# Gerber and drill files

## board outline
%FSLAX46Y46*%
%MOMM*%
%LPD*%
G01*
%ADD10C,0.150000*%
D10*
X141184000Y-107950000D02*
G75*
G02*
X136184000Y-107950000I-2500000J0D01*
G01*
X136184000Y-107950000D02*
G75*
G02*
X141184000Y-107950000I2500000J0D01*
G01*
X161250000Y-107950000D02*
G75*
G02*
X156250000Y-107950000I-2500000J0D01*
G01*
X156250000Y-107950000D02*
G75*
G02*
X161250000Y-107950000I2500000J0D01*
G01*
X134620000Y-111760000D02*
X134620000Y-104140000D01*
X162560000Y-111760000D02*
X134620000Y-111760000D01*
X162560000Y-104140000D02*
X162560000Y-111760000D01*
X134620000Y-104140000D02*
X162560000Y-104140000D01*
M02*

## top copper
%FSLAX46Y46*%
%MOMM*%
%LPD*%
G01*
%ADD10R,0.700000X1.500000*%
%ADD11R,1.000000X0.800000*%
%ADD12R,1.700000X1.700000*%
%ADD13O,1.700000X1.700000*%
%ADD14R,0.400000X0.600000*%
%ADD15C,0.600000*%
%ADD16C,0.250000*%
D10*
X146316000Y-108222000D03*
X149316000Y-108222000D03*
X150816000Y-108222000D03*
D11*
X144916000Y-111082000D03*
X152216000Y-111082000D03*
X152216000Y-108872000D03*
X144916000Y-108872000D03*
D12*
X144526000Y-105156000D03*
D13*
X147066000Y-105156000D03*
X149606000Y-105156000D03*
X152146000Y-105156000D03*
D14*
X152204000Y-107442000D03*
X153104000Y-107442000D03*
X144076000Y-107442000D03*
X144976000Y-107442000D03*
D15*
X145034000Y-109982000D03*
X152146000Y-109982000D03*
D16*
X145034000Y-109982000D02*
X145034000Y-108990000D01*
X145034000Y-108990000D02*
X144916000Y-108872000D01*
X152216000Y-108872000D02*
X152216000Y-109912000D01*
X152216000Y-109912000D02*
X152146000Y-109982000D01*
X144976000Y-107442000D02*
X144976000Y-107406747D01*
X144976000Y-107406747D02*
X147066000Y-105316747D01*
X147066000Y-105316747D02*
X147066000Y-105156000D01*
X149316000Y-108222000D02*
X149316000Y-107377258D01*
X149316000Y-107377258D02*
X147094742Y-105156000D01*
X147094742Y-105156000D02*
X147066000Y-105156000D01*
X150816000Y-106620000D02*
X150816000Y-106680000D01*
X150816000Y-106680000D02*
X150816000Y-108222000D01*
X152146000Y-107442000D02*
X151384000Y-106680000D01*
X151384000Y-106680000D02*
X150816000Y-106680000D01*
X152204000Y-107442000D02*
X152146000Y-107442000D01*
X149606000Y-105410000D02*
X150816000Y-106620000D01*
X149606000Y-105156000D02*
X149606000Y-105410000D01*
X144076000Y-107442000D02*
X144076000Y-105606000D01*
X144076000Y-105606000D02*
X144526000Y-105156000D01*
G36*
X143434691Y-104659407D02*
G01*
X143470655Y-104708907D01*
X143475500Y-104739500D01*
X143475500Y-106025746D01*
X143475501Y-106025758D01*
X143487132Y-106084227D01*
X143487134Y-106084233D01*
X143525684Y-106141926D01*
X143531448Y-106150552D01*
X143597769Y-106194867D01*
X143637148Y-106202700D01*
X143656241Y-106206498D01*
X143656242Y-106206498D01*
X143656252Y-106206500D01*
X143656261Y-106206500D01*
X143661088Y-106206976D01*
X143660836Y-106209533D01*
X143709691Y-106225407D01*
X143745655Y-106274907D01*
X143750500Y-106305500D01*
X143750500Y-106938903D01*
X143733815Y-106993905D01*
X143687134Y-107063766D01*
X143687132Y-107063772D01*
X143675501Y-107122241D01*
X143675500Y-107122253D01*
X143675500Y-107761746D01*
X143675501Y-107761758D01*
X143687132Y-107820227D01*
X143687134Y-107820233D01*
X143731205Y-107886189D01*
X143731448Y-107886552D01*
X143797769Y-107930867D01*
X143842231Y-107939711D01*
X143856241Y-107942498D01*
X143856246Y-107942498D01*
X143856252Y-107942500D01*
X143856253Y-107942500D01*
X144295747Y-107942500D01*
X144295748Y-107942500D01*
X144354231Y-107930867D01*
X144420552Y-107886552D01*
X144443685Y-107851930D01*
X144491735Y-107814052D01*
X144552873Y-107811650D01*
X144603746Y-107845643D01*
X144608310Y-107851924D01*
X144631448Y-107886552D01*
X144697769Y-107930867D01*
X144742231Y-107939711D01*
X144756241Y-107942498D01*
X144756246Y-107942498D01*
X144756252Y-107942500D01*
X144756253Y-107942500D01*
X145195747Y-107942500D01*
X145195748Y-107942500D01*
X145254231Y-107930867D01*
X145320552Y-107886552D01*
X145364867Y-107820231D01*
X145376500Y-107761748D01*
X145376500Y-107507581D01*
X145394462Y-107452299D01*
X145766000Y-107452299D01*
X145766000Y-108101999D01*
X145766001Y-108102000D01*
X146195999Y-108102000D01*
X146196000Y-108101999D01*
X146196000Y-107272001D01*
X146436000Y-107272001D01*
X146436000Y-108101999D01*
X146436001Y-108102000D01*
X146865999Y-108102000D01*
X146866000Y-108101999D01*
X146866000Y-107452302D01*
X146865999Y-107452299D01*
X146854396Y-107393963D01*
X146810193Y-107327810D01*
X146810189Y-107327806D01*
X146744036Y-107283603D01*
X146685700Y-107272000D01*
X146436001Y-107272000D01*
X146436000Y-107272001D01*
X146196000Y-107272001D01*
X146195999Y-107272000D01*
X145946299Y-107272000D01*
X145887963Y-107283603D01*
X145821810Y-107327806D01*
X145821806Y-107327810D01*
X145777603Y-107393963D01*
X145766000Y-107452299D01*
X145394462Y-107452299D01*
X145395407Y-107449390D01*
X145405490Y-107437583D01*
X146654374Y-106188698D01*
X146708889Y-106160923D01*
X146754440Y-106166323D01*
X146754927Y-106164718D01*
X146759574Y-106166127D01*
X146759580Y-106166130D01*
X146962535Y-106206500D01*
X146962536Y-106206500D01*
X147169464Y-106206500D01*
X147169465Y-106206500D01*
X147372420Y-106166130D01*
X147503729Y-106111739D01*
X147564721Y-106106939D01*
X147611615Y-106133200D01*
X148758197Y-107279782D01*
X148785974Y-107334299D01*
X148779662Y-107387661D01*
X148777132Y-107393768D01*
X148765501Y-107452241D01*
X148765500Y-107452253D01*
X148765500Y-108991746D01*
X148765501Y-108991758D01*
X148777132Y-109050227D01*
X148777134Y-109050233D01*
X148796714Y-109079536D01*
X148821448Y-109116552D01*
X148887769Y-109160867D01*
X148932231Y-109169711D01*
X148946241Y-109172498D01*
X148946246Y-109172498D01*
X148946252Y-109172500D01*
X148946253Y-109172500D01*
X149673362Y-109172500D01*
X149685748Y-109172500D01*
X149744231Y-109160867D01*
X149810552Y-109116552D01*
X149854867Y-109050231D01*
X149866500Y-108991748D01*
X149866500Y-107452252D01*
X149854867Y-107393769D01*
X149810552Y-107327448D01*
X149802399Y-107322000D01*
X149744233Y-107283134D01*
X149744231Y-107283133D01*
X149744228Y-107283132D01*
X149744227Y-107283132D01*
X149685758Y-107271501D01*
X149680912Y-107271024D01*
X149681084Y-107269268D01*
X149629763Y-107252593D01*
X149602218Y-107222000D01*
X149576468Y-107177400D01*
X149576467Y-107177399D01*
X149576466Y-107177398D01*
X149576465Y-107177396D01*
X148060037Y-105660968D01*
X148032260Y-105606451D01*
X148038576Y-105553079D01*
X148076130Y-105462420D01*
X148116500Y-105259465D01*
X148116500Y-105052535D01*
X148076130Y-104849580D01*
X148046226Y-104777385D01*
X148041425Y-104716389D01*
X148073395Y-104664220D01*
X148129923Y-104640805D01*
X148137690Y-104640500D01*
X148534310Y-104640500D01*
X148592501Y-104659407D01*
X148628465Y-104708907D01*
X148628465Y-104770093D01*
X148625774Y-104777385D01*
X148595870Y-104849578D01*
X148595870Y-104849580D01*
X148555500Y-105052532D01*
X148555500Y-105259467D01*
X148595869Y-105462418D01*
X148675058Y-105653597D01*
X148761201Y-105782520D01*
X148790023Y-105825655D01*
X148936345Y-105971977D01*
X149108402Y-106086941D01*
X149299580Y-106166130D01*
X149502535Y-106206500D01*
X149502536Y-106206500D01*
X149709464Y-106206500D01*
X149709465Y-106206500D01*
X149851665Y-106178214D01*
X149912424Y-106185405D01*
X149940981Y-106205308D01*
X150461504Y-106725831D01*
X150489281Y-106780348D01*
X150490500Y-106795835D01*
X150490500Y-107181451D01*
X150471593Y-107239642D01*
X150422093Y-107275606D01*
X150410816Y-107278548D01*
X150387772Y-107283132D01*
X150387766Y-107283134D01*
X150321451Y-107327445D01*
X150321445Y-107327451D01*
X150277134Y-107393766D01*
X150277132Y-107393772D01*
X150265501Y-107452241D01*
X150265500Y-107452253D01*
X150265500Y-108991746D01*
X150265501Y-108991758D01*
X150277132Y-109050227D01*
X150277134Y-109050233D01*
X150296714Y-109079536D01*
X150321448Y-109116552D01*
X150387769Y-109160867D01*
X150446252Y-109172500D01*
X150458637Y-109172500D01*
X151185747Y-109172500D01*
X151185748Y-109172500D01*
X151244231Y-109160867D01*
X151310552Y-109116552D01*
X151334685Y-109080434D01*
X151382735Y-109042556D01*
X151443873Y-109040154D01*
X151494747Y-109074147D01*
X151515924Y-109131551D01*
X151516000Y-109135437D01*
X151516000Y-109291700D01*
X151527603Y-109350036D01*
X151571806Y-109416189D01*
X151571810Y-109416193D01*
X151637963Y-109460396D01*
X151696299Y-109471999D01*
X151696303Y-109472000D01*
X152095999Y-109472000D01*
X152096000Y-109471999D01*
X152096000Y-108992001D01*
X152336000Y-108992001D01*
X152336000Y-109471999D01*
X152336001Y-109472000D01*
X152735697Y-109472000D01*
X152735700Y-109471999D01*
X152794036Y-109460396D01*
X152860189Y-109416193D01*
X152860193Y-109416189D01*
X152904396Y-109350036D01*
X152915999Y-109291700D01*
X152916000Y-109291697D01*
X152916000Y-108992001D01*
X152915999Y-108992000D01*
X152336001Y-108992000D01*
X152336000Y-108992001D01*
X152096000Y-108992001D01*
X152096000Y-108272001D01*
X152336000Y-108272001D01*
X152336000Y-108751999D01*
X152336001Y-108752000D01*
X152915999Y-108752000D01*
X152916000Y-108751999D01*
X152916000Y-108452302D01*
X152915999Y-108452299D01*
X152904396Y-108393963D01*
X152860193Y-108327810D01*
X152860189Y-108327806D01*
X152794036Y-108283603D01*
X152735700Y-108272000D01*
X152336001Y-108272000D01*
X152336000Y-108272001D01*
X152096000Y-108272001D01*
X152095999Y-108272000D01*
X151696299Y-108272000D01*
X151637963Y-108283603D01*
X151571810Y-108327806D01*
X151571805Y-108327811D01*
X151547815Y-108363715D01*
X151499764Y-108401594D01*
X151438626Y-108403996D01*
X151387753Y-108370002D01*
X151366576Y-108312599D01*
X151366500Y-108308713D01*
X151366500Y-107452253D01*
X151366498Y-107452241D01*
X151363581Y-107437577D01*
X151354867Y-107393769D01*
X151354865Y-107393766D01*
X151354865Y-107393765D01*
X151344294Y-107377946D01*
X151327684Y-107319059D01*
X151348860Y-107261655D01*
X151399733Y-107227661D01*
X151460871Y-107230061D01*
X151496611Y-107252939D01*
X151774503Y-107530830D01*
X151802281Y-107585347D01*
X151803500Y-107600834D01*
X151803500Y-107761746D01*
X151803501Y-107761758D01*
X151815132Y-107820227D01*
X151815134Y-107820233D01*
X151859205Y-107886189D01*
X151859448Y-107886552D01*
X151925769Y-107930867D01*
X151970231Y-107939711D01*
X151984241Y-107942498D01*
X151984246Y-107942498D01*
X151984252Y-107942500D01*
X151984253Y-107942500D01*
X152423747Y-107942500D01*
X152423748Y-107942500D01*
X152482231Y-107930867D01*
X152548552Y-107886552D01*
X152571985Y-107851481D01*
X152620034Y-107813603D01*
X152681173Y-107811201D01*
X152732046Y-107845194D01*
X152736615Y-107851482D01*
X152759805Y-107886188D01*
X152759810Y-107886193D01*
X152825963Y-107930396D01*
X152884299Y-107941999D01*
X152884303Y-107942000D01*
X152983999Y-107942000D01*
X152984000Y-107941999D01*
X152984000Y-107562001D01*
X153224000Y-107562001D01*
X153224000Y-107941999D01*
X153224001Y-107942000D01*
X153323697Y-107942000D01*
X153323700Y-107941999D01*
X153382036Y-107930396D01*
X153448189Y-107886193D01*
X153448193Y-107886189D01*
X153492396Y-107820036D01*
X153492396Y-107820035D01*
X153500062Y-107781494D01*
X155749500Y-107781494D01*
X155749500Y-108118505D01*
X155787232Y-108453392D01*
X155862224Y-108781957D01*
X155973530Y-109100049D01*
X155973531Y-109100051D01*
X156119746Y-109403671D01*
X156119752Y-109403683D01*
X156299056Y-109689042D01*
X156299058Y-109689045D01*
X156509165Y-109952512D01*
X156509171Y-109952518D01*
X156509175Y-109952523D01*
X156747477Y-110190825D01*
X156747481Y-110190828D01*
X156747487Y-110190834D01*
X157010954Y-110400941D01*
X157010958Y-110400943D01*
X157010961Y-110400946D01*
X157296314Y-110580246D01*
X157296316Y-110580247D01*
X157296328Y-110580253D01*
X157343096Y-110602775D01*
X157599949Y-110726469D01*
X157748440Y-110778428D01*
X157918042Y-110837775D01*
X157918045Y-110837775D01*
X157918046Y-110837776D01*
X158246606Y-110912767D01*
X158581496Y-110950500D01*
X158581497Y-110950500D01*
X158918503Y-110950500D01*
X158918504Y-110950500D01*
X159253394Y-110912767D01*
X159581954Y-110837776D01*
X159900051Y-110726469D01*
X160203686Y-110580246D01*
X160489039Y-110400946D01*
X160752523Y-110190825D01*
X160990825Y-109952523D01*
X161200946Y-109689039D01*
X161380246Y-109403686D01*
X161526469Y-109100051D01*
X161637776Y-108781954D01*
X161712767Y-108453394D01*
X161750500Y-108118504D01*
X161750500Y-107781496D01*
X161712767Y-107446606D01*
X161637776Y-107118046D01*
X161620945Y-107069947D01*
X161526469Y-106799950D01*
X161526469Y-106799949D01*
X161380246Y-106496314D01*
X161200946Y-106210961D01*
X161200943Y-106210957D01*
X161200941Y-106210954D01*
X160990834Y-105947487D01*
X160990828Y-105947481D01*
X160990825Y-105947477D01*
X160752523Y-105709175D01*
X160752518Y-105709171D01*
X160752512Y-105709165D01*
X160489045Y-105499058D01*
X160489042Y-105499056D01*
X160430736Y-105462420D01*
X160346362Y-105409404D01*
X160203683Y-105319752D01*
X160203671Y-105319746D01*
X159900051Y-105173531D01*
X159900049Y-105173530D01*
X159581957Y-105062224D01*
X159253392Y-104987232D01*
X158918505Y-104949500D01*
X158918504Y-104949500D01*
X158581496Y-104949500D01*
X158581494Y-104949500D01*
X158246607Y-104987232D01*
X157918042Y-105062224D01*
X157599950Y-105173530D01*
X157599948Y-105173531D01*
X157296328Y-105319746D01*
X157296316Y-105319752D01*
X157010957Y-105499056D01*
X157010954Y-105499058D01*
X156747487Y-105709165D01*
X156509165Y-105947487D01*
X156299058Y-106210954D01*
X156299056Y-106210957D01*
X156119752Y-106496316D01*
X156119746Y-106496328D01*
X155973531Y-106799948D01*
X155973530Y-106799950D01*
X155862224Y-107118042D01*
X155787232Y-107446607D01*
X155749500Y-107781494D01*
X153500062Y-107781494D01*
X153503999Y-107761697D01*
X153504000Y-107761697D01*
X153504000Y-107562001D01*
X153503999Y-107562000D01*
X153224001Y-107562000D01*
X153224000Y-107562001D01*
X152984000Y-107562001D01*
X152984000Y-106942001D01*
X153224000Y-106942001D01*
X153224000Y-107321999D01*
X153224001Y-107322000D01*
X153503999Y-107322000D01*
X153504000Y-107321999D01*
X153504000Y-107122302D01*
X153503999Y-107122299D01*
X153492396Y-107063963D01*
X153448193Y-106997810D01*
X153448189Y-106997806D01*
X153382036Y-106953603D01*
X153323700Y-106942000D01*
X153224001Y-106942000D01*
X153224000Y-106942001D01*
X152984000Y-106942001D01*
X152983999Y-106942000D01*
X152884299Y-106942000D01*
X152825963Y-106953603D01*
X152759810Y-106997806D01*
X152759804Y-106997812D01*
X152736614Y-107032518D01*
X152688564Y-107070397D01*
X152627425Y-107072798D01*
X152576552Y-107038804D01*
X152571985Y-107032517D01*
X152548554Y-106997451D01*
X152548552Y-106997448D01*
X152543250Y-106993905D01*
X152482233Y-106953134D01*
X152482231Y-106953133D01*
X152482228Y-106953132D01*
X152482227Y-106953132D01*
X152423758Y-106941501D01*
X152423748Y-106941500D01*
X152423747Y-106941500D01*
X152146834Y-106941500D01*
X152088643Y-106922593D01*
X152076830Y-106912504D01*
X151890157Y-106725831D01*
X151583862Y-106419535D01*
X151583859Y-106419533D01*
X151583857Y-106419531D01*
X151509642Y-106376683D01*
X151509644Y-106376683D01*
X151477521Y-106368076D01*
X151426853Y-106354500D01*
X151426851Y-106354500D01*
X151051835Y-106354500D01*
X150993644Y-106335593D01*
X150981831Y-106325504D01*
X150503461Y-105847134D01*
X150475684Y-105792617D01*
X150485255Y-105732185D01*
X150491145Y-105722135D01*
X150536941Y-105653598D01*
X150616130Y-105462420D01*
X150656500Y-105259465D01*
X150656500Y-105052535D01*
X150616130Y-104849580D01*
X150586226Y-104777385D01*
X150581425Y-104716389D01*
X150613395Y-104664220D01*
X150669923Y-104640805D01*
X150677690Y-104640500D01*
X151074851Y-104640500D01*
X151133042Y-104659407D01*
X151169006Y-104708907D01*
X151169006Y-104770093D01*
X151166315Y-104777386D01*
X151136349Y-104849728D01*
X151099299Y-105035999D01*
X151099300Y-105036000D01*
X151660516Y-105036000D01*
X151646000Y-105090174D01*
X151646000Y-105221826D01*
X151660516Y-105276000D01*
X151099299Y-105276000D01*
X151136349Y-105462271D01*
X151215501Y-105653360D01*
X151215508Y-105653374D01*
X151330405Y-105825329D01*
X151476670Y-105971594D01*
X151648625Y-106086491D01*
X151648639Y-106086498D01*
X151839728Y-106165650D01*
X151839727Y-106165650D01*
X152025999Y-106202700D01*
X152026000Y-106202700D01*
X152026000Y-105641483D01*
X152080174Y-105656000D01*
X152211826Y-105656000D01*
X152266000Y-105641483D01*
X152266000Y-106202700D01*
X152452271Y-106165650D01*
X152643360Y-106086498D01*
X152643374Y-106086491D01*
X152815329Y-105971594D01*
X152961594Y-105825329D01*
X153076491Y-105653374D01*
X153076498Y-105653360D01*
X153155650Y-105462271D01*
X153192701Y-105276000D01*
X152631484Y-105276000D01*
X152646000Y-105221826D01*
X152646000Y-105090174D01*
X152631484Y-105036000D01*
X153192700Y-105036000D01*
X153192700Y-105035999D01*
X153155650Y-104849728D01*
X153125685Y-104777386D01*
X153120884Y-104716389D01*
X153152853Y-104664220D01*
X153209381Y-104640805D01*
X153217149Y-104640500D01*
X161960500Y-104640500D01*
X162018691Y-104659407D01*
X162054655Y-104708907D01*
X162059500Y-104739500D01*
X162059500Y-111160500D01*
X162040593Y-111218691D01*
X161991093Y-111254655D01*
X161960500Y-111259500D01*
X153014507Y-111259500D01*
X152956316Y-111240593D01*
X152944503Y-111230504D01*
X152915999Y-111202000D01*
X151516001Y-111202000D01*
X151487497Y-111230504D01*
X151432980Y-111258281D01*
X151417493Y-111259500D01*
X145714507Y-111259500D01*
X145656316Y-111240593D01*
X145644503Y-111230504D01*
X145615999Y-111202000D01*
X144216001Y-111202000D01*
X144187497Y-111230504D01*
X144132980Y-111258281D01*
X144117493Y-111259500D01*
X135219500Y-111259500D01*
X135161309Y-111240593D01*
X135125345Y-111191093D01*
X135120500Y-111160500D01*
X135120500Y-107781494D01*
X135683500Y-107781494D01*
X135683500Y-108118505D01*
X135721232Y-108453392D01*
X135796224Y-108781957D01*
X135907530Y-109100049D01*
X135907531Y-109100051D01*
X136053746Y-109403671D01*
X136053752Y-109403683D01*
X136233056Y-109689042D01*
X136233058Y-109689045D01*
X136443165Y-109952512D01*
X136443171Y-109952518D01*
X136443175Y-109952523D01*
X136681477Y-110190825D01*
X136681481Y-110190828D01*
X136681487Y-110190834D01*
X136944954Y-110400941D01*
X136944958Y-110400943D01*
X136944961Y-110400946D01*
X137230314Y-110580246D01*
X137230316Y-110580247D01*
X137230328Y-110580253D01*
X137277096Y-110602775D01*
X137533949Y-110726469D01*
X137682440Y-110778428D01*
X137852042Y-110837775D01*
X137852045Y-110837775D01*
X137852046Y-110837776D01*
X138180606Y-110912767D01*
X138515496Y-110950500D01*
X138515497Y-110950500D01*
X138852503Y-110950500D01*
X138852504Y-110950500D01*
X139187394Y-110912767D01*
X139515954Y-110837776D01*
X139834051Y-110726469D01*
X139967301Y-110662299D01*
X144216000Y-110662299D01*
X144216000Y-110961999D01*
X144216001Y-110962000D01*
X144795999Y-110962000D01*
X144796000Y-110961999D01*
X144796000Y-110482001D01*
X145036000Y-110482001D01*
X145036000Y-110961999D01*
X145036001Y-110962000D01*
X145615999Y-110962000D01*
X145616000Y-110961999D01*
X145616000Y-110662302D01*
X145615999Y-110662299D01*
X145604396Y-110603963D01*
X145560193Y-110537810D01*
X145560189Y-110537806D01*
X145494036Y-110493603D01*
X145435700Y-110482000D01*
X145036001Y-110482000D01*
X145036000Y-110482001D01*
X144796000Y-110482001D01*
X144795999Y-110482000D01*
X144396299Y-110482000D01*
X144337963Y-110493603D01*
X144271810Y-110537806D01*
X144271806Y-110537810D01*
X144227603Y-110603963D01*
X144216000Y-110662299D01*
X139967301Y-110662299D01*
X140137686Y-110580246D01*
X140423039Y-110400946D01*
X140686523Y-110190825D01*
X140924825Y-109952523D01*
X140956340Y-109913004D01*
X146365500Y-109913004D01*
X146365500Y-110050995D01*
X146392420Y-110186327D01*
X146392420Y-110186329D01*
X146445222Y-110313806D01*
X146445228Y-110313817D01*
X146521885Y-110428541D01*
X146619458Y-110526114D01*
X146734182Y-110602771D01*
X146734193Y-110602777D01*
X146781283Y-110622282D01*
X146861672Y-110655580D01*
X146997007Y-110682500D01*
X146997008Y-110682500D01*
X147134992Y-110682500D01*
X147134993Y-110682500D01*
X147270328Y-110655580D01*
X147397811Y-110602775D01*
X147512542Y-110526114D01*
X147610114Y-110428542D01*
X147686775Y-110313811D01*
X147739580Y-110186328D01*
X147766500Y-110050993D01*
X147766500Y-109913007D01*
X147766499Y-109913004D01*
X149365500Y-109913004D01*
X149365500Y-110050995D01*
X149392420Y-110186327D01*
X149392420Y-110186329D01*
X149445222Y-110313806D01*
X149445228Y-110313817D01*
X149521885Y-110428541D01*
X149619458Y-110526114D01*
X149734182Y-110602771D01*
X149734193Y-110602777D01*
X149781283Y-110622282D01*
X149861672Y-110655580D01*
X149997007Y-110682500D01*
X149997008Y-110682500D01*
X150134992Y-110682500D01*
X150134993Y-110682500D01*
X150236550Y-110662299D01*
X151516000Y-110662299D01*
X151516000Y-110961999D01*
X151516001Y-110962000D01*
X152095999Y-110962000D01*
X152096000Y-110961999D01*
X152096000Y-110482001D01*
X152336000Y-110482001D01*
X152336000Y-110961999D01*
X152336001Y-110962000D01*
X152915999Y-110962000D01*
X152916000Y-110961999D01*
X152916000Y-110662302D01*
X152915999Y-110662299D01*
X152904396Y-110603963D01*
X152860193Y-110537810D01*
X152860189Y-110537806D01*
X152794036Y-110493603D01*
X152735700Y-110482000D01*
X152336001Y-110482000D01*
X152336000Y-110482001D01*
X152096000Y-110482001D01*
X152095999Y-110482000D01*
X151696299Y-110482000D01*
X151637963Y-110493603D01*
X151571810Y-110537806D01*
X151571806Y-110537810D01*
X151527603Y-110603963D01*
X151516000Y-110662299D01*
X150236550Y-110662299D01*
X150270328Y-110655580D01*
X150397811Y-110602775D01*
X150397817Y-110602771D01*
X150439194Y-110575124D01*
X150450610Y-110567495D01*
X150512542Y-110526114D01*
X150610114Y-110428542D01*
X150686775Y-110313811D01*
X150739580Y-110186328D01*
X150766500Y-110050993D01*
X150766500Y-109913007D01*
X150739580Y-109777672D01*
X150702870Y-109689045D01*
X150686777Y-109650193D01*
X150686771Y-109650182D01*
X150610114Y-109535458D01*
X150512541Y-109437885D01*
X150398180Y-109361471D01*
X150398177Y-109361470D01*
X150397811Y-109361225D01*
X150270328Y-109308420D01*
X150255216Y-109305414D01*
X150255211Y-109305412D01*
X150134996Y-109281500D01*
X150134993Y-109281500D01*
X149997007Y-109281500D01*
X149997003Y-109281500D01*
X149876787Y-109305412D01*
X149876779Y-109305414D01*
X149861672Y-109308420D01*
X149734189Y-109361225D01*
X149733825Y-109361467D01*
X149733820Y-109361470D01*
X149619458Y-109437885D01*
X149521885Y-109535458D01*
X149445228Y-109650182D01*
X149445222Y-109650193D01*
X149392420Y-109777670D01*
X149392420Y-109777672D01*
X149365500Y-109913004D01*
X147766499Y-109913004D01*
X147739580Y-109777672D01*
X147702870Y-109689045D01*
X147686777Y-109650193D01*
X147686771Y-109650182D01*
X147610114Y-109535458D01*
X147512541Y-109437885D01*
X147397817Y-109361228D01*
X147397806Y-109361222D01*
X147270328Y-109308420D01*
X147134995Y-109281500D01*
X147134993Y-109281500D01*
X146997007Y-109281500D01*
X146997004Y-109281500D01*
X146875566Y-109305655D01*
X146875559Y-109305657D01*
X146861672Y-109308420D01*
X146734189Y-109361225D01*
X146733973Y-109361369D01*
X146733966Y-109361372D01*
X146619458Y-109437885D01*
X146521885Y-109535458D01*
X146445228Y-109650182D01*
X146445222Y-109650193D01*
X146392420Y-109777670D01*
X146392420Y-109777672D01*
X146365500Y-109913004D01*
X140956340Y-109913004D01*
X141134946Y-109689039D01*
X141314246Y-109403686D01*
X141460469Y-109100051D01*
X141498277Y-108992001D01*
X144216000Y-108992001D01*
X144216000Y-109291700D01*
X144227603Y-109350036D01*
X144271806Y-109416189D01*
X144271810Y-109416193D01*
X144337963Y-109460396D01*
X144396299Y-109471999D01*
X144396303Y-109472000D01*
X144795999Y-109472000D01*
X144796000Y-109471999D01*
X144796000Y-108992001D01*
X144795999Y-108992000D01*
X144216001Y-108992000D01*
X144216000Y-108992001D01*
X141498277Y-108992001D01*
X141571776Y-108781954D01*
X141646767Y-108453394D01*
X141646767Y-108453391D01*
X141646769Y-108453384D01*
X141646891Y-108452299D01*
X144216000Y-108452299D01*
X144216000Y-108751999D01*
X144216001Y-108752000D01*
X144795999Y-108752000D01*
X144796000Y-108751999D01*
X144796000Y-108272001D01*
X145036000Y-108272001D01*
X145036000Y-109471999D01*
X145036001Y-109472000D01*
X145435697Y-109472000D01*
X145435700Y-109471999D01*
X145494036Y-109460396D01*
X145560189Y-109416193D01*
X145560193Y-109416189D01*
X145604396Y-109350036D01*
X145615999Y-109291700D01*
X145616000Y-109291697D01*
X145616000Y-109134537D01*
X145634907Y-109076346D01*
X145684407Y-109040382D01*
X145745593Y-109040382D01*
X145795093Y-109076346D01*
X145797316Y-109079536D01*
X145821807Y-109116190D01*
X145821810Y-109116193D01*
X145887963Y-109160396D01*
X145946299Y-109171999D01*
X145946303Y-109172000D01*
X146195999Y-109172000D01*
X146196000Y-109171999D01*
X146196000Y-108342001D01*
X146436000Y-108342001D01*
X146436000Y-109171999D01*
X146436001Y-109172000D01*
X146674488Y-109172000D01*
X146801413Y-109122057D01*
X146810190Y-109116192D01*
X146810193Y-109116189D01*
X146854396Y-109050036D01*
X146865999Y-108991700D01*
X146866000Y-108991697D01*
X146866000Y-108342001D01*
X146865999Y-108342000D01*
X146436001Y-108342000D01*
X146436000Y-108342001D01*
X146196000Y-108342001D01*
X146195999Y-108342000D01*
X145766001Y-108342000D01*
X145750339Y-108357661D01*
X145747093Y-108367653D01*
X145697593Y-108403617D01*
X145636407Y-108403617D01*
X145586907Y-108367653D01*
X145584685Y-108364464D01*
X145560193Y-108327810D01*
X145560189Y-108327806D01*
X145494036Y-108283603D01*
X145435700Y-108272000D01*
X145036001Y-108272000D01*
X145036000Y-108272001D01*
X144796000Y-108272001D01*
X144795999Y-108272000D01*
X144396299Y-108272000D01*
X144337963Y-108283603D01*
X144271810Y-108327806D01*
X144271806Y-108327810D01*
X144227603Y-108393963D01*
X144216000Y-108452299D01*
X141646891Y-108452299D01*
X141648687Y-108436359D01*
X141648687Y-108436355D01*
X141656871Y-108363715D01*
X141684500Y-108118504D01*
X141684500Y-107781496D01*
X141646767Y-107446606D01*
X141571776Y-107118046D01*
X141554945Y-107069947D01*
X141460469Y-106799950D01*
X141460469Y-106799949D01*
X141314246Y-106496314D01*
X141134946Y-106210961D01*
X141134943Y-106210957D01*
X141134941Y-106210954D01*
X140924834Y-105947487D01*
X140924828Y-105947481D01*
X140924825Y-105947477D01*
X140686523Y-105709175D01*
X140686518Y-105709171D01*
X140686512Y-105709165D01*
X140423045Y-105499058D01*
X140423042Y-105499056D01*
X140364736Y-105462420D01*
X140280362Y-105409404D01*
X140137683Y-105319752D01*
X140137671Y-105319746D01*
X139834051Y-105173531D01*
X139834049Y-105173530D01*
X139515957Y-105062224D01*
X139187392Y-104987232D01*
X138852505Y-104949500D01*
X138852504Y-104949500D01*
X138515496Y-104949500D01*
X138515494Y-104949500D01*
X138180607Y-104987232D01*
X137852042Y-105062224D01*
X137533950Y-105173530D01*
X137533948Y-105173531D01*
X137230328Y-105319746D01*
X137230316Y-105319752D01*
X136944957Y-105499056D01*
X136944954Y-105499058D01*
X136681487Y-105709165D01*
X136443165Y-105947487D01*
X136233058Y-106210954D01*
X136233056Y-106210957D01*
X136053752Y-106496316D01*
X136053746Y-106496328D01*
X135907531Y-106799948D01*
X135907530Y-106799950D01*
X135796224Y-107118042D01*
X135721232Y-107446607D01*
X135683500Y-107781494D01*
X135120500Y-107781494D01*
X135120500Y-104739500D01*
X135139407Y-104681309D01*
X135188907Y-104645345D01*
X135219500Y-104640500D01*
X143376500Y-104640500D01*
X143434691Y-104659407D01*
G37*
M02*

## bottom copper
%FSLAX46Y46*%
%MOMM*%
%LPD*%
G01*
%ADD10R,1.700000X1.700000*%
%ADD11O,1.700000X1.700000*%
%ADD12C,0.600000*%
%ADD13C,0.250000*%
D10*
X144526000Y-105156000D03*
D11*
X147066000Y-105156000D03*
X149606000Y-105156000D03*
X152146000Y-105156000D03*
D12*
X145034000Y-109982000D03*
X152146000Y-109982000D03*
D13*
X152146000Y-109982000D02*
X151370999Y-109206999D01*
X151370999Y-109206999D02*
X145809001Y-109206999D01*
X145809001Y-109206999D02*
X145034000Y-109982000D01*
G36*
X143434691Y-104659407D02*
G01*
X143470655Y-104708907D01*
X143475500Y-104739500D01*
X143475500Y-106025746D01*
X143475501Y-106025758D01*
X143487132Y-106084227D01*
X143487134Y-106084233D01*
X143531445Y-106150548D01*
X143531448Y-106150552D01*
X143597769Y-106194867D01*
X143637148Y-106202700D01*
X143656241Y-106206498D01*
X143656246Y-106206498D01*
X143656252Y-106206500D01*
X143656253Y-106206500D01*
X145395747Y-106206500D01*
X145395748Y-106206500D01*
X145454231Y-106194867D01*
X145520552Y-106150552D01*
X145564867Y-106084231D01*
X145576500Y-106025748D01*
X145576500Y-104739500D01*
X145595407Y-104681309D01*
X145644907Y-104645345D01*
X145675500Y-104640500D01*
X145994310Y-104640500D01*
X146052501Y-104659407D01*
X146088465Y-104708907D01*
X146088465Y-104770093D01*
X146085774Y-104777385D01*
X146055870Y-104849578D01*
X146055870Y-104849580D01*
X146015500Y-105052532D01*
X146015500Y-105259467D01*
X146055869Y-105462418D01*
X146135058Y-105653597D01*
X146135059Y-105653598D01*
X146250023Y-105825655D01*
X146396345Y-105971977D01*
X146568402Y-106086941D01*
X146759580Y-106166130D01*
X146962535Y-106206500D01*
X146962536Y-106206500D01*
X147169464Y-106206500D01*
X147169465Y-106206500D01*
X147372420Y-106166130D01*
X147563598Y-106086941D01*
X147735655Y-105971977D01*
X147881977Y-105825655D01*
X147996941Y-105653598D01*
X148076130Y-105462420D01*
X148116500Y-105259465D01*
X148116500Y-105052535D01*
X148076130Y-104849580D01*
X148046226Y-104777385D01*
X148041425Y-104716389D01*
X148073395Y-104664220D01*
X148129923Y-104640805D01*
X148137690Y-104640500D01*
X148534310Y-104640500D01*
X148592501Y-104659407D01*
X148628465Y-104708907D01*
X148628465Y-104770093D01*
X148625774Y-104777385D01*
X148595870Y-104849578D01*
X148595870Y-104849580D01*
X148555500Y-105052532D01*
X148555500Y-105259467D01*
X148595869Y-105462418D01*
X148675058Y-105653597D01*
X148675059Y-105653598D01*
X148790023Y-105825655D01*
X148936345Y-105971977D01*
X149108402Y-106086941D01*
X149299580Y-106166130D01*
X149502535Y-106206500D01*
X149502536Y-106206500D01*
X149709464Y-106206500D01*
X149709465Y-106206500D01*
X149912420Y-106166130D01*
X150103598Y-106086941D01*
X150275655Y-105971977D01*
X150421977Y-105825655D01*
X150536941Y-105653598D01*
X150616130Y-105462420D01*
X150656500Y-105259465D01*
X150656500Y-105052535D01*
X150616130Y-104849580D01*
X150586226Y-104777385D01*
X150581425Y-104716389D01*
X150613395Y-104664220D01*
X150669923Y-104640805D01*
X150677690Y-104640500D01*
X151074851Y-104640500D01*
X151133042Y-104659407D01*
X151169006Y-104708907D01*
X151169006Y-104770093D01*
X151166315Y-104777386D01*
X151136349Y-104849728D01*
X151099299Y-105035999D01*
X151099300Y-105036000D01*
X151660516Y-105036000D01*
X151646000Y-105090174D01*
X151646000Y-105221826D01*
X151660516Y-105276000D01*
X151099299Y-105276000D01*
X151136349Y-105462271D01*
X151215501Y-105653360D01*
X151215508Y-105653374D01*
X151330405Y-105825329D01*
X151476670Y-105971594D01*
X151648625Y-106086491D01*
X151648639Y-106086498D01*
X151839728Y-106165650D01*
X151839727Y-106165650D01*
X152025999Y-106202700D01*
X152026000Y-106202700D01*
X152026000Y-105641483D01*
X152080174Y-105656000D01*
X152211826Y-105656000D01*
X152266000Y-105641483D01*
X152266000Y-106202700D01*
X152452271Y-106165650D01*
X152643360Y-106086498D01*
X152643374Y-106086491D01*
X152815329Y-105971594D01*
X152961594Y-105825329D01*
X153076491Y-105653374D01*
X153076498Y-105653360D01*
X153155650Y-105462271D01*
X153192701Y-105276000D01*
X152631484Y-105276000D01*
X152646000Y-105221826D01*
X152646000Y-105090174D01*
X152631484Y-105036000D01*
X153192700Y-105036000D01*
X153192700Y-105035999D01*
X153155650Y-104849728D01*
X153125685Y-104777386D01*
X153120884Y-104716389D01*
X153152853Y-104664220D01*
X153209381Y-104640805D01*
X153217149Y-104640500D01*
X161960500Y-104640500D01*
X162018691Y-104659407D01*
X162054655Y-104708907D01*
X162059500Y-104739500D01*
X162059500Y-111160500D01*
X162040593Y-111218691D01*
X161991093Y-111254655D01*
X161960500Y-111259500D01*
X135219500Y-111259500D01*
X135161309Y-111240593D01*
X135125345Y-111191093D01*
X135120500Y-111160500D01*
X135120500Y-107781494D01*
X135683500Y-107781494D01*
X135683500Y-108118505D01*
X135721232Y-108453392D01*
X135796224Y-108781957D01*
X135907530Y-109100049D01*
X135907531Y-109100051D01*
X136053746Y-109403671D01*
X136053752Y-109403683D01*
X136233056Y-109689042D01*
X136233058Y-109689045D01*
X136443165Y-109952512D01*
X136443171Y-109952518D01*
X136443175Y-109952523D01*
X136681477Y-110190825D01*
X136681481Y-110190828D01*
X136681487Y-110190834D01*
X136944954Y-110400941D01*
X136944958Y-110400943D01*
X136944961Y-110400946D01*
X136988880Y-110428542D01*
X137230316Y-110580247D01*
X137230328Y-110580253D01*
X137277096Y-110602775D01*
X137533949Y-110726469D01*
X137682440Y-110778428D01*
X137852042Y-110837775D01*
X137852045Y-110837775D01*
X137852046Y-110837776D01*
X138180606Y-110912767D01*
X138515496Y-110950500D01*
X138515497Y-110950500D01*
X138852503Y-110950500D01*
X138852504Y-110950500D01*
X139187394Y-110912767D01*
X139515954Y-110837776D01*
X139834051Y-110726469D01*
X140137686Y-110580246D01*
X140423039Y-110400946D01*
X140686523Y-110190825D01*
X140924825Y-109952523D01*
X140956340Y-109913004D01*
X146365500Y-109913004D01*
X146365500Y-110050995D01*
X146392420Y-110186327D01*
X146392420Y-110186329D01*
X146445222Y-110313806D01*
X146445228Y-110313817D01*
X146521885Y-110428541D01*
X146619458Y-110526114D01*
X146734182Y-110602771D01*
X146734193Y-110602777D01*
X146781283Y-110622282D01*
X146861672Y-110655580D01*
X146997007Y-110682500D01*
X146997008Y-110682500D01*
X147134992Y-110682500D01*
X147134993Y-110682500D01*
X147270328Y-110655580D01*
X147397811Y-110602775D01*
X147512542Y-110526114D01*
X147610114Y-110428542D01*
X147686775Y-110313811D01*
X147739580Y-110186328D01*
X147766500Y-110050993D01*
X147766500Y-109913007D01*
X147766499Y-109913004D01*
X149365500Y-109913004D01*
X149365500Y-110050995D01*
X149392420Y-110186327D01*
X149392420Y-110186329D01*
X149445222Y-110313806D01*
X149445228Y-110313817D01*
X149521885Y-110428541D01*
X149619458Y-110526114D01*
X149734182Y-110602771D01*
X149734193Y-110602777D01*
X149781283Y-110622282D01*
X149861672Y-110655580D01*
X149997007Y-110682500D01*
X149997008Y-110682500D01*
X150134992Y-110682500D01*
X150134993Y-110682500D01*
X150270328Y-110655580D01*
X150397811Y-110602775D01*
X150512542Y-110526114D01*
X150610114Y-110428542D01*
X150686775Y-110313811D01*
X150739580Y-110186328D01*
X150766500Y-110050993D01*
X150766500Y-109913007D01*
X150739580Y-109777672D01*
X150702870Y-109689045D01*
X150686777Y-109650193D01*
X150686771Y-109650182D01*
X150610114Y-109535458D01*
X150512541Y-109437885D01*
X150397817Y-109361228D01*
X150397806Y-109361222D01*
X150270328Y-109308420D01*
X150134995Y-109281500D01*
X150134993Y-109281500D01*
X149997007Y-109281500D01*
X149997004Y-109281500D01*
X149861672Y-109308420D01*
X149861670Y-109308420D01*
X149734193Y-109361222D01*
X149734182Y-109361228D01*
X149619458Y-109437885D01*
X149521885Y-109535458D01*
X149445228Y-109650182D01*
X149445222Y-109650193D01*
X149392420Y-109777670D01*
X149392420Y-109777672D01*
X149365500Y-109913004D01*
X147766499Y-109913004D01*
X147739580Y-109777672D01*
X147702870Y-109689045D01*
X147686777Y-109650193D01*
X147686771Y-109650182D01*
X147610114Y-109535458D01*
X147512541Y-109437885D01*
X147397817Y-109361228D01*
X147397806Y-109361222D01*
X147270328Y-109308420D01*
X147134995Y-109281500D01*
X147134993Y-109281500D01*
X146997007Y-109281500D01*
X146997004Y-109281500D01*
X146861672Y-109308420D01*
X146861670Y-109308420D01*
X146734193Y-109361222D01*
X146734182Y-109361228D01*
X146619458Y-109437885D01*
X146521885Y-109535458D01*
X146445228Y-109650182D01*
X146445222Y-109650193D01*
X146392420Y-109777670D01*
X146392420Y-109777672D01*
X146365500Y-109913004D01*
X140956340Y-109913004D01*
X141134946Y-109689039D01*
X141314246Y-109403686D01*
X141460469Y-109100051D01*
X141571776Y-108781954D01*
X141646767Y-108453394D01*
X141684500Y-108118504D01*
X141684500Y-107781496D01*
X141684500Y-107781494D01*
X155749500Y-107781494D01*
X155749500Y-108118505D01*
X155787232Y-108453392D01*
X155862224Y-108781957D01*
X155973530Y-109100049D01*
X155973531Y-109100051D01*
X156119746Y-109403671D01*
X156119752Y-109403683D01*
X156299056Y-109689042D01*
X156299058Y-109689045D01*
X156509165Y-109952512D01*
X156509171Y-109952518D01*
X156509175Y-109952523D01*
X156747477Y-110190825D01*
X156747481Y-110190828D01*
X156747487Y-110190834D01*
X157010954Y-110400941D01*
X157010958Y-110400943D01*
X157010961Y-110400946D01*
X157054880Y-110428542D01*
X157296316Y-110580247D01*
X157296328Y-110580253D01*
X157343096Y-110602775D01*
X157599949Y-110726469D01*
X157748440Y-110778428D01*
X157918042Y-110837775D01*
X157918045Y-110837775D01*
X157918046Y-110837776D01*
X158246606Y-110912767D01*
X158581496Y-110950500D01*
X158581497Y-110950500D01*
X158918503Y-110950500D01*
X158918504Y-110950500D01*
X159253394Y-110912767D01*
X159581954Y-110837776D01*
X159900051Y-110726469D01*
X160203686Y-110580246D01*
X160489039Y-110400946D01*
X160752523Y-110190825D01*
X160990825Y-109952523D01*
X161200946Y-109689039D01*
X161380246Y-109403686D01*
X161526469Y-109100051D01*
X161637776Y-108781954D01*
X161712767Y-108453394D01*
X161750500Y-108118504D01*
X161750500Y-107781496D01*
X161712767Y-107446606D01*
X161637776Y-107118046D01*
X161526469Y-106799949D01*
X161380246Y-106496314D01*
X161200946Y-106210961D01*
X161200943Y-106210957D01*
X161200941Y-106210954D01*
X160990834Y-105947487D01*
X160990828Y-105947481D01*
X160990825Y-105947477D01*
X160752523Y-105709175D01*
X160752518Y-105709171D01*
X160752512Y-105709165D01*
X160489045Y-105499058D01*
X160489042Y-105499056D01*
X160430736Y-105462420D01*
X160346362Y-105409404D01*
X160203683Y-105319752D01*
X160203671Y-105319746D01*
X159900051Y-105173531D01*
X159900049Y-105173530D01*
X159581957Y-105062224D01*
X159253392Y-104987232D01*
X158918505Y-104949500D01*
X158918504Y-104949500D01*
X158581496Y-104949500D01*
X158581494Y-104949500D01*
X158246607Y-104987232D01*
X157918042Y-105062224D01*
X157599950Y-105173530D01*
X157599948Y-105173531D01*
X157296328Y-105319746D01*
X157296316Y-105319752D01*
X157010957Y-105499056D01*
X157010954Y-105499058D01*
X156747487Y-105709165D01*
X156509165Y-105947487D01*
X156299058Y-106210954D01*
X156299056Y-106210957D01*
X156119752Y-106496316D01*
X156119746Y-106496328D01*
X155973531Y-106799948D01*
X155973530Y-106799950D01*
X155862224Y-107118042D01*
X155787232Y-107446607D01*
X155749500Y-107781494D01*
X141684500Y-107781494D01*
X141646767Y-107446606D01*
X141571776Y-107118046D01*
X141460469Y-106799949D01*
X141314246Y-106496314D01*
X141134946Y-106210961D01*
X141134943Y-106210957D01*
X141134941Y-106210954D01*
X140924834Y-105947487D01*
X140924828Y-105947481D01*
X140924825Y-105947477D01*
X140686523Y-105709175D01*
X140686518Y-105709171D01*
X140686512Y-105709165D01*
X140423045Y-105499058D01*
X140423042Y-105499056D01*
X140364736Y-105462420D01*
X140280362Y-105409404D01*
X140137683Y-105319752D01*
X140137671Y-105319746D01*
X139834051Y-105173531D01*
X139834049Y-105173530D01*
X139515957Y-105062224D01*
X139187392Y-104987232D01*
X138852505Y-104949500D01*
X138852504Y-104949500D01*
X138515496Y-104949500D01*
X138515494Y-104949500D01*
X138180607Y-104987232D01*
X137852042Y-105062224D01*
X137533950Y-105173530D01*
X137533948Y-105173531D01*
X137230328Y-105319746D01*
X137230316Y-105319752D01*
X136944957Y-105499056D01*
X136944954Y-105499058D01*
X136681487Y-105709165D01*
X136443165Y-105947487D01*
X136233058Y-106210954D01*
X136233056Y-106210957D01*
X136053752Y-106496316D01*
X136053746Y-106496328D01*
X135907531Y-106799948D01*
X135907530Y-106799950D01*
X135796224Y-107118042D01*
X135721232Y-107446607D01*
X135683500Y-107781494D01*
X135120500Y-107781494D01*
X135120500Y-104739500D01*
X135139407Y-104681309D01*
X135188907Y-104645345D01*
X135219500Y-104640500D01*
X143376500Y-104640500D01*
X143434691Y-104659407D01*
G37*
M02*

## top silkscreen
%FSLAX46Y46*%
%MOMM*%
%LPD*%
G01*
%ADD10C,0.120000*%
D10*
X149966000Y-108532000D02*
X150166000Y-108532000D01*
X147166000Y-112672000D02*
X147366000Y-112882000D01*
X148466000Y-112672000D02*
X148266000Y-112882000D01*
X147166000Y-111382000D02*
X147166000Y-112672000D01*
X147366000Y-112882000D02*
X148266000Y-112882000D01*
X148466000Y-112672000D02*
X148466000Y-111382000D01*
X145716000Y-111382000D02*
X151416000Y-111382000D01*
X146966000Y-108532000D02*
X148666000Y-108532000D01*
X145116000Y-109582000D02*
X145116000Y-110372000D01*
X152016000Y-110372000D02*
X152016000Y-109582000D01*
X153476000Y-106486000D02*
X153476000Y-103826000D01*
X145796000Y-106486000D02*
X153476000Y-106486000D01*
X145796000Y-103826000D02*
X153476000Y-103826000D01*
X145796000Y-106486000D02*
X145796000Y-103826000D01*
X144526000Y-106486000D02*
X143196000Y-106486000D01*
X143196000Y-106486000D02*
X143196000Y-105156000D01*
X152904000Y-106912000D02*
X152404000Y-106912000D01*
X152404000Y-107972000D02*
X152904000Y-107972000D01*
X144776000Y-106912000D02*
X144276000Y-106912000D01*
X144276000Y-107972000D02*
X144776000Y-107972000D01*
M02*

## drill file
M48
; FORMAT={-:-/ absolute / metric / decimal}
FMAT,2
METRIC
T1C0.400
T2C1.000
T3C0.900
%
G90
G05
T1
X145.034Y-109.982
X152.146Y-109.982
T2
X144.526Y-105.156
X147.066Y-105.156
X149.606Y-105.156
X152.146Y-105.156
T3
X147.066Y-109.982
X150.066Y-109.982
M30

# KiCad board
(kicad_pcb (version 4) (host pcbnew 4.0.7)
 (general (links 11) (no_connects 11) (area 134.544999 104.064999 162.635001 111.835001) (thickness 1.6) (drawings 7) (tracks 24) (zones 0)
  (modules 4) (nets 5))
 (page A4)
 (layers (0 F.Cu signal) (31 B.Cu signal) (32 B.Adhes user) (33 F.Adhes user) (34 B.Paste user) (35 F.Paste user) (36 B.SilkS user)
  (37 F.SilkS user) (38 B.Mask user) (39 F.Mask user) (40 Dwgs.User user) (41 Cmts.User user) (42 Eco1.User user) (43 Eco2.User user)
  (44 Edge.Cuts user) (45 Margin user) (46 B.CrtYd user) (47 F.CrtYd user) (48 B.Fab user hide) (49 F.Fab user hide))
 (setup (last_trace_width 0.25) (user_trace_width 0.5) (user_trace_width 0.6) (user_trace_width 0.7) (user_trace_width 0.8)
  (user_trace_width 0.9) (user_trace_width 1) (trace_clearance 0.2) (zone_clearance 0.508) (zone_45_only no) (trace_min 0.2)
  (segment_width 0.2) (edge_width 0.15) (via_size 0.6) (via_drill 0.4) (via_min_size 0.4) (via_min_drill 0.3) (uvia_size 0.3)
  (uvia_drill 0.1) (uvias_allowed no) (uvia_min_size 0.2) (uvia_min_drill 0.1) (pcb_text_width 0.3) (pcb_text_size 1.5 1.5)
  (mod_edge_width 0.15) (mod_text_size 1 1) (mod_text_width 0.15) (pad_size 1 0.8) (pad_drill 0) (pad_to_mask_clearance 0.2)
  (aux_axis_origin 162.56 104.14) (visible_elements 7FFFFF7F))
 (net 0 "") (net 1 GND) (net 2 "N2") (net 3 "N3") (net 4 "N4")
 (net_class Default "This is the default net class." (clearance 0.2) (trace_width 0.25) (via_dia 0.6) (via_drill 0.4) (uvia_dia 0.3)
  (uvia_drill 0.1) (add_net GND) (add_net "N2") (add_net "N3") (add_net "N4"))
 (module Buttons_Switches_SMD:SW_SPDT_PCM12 (layer F.Cu) (at 148.566 109.652)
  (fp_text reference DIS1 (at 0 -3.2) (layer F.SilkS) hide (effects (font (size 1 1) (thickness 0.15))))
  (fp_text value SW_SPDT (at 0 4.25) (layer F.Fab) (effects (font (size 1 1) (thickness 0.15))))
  (fp_line (start 1.4 -1.12) (end 1.6 -1.12) (layer F.SilkS) (width 0.12))
  (fp_line (start -1.4 3.02) (end -1.2 3.23) (layer F.SilkS) (width 0.12))
  (fp_line (start -0.1 3.02) (end -0.3 3.23) (layer F.SilkS) (width 0.12))
  (fp_line (start -1.4 1.73) (end -1.4 3.02) (layer F.SilkS) (width 0.12))
  (fp_line (start -1.2 3.23) (end -0.3 3.23) (layer F.SilkS) (width 0.12))
  (fp_line (start -0.1 3.02) (end -0.1 1.73) (layer F.SilkS) (width 0.12))
  (fp_line (start -2.85 1.73) (end 2.85 1.73) (layer F.SilkS) (width 0.12))
  (fp_line (start -1.6 -1.12) (end 0.1 -1.12) (layer F.SilkS) (width 0.12))
  (fp_line (start -3.45 -0.07) (end -3.45 0.72) (layer F.SilkS) (width 0.12))
  (fp_line (start 3.45 0.72) (end 3.45 -0.07) (layer F.SilkS) (width 0.12))
  (pad "" np_thru_hole circle (at -1.5 0.33) (size 0.9 0.9) (drill 0.9) (layers *.Cu *.Mask))
  (pad "" np_thru_hole circle (at 1.5 0.33) (size 0.9 0.9) (drill 0.9) (layers *.Cu *.Mask))
  (pad 1 smd rect (at -2.25 -1.43) (size 0.7 1.5) (layers F.Cu F.Paste F.Mask) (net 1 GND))
  (pad 2 smd rect (at 0.75 -1.43) (size 0.7 1.5) (layers F.Cu F.Paste F.Mask) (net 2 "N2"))
  (pad 3 smd rect (at 2.25 -1.43) (size 0.7 1.5) (layers F.Cu F.Paste F.Mask) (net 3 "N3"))
  (pad 1 smd rect (at -3.65 1.43) (size 1 0.8) (layers F.Cu F.Paste F.Mask) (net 1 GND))
  (pad 1 smd rect (at 3.65 1.43) (size 1 0.8) (layers F.Cu F.Paste F.Mask) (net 1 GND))
  (pad 1 smd rect (at 3.65 -0.78) (size 1 0.8) (layers F.Cu F.Paste F.Mask) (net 1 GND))
  (pad 1 smd rect (at -3.65 -0.78) (size 1 0.8) (layers F.Cu F.Paste F.Mask) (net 1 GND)))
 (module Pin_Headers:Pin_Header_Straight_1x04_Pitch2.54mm (layer F.Cu) (at 144.526 105.156 90)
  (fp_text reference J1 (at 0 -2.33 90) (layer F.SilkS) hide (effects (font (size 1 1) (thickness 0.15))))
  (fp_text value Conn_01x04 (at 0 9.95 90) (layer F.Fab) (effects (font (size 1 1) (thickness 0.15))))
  (fp_line (start -1.33 8.95) (end 1.33 8.95) (layer F.SilkS) (width 0.12))
  (fp_line (start -1.33 1.27) (end -1.33 8.95) (layer F.SilkS) (width 0.12))
  (fp_line (start 1.33 1.27) (end 1.33 8.95) (layer F.SilkS) (width 0.12))
  (fp_line (start -1.33 1.27) (end 1.33 1.27) (layer F.SilkS) (width 0.12))
  (fp_line (start -1.33 0) (end -1.33 -1.33) (layer F.SilkS) (width 0.12))
  (fp_line (start -1.33 -1.33) (end 0 -1.33) (layer F.SilkS) (width 0.12))
  (pad 1 thru_hole rect (at 0 0 90) (size 1.7 1.7) (drill 1) (layers *.Cu *.Mask) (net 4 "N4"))
  (pad 2 thru_hole oval (at 0 2.54 90) (size 1.7 1.7) (drill 1) (layers *.Cu *.Mask) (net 2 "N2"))
  (pad 3 thru_hole oval (at 0 5.08 90) (size 1.7 1.7) (drill 1) (layers *.Cu *.Mask) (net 3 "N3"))
  (pad 4 thru_hole oval (at 0 7.62 90) (size 1.7 1.7) (drill 1) (layers *.Cu *.Mask) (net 1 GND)))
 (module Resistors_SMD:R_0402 (layer F.Cu) (at 152.654 107.442)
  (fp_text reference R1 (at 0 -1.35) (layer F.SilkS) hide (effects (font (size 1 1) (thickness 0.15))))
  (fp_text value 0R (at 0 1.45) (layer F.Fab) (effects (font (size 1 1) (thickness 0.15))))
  (fp_line (start 0.25 -0.53) (end -0.25 -0.53) (layer F.SilkS) (width 0.12))
  (fp_line (start -0.25 0.53) (end 0.25 0.53) (layer F.SilkS) (width 0.12))
  (pad 1 smd rect (at -0.45 0) (size 0.4 0.6) (layers F.Cu F.Paste F.Mask) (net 3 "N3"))
  (pad 2 smd rect (at 0.45 0) (size 0.4 0.6) (layers F.Cu F.Paste F.Mask) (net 1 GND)))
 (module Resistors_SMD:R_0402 (layer F.Cu) (at 144.526 107.442)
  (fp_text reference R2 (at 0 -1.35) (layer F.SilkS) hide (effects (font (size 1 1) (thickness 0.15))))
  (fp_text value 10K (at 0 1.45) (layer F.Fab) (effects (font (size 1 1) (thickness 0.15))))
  (fp_line (start 0.25 -0.53) (end -0.25 -0.53) (layer F.SilkS) (width 0.12))
  (fp_line (start -0.25 0.53) (end 0.25 0.53) (layer F.SilkS) (width 0.12))
  (pad 1 smd rect (at -0.45 0) (size 0.4 0.6) (layers F.Cu F.Paste F.Mask) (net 4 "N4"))
  (pad 2 smd rect (at 0.45 0) (size 0.4 0.6) (layers F.Cu F.Paste F.Mask) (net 2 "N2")))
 (gr_circle (center 138.684 107.95) (end 138.684 110.45) (layer Edge.Cuts) (width 0.15))
 (gr_circle (center 158.75 107.95) (end 158.75 110.45) (layer Edge.Cuts) (width 0.15))
 (gr_line (start 134.62 111.76) (end 134.62 104.14) (layer Edge.Cuts) (width 0.15))
 (gr_line (start 162.56 111.76) (end 134.62 111.76) (layer Edge.Cuts) (width 0.15))
 (gr_line (start 162.56 104.14) (end 162.56 111.76) (layer Edge.Cuts) (width 0.15))
 (gr_line (start 134.62 104.14) (end 162.56 104.14) (layer Edge.Cuts) (width 0.15))
 (segment (start 145.034 109.982) (end 145.034 108.99) (width 0.25) (layer F.Cu) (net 1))
 (segment (start 145.034 108.99) (end 144.916 108.872) (width 0.25) (layer F.Cu) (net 1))
 (segment (start 152.146 109.982) (end 151.370999 109.206999) (width 0.25) (layer B.Cu) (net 1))
 (segment (start 151.370999 109.206999) (end 145.809001 109.206999) (width 0.25) (layer B.Cu) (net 1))
 (segment (start 145.809001 109.206999) (end 145.034 109.982) (width 0.25) (layer B.Cu) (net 1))
 (via (at 145.034 109.982) (size 0.6) (drill 0.4) (layers F.Cu B.Cu) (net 1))
 (segment (start 152.216 108.872) (end 152.216 109.912) (width 0.25) (layer F.Cu) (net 1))
 (segment (start 152.216 109.912) (end 152.146 109.982) (width 0.25) (layer F.Cu) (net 1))
 (via (at 152.146 109.982) (size 0.6) (drill 0.4) (layers F.Cu B.Cu) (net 1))
 (segment (start 144.976 107.442) (end 144.976 107.406747) (width 0.25) (layer F.Cu) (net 2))
 (segment (start 144.976 107.406747) (end 147.066 105.316747) (width 0.25) (layer F.Cu) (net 2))
 (segment (start 147.066 105.316747) (end 147.066 105.156) (width 0.25) (layer F.Cu) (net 2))
 (segment (start 149.316 108.222) (end 149.316 107.377258) (width 0.25) (layer F.Cu) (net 2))
 (segment (start 149.316 107.377258) (end 147.094742 105.156) (width 0.25) (layer F.Cu) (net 2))
 (segment (start 147.094742 105.156) (end 147.066 105.156) (width 0.25) (layer F.Cu) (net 2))
 (segment (start 150.816 106.62) (end 150.816 106.68) (width 0.25) (layer F.Cu) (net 3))
 (segment (start 150.816 106.68) (end 150.816 108.222) (width 0.25) (layer F.Cu) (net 3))
 (segment (start 152.146 107.442) (end 151.384 106.68) (width 0.25) (layer F.Cu) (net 3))
 (segment (start 151.384 106.68) (end 150.816 106.68) (width 0.25) (layer F.Cu) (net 3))
 (segment (start 152.204 107.442) (end 152.146 107.442) (width 0.25) (layer F.Cu) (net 3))
 (segment (start 149.606 105.41) (end 150.816 106.62) (width 0.25) (layer F.Cu) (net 3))
 (segment (start 149.606 105.156) (end 149.606 105.41) (width 0.25) (layer F.Cu) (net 3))
 (segment (start 144.076 107.442) (end 144.076 105.606) (width 0.25) (layer F.Cu) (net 4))
 (segment (start 144.076 105.606) (end 144.526 105.156) (width 0.25) (layer F.Cu) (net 4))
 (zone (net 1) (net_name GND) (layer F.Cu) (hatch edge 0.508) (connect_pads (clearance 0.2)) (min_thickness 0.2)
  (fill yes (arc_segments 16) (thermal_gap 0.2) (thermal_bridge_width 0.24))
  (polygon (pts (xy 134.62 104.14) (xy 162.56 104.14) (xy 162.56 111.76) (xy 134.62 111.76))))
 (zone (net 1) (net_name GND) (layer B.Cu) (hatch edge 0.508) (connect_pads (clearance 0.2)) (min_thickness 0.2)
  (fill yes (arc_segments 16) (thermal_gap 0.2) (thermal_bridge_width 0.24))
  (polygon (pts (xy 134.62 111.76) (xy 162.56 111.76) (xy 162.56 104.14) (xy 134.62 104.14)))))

